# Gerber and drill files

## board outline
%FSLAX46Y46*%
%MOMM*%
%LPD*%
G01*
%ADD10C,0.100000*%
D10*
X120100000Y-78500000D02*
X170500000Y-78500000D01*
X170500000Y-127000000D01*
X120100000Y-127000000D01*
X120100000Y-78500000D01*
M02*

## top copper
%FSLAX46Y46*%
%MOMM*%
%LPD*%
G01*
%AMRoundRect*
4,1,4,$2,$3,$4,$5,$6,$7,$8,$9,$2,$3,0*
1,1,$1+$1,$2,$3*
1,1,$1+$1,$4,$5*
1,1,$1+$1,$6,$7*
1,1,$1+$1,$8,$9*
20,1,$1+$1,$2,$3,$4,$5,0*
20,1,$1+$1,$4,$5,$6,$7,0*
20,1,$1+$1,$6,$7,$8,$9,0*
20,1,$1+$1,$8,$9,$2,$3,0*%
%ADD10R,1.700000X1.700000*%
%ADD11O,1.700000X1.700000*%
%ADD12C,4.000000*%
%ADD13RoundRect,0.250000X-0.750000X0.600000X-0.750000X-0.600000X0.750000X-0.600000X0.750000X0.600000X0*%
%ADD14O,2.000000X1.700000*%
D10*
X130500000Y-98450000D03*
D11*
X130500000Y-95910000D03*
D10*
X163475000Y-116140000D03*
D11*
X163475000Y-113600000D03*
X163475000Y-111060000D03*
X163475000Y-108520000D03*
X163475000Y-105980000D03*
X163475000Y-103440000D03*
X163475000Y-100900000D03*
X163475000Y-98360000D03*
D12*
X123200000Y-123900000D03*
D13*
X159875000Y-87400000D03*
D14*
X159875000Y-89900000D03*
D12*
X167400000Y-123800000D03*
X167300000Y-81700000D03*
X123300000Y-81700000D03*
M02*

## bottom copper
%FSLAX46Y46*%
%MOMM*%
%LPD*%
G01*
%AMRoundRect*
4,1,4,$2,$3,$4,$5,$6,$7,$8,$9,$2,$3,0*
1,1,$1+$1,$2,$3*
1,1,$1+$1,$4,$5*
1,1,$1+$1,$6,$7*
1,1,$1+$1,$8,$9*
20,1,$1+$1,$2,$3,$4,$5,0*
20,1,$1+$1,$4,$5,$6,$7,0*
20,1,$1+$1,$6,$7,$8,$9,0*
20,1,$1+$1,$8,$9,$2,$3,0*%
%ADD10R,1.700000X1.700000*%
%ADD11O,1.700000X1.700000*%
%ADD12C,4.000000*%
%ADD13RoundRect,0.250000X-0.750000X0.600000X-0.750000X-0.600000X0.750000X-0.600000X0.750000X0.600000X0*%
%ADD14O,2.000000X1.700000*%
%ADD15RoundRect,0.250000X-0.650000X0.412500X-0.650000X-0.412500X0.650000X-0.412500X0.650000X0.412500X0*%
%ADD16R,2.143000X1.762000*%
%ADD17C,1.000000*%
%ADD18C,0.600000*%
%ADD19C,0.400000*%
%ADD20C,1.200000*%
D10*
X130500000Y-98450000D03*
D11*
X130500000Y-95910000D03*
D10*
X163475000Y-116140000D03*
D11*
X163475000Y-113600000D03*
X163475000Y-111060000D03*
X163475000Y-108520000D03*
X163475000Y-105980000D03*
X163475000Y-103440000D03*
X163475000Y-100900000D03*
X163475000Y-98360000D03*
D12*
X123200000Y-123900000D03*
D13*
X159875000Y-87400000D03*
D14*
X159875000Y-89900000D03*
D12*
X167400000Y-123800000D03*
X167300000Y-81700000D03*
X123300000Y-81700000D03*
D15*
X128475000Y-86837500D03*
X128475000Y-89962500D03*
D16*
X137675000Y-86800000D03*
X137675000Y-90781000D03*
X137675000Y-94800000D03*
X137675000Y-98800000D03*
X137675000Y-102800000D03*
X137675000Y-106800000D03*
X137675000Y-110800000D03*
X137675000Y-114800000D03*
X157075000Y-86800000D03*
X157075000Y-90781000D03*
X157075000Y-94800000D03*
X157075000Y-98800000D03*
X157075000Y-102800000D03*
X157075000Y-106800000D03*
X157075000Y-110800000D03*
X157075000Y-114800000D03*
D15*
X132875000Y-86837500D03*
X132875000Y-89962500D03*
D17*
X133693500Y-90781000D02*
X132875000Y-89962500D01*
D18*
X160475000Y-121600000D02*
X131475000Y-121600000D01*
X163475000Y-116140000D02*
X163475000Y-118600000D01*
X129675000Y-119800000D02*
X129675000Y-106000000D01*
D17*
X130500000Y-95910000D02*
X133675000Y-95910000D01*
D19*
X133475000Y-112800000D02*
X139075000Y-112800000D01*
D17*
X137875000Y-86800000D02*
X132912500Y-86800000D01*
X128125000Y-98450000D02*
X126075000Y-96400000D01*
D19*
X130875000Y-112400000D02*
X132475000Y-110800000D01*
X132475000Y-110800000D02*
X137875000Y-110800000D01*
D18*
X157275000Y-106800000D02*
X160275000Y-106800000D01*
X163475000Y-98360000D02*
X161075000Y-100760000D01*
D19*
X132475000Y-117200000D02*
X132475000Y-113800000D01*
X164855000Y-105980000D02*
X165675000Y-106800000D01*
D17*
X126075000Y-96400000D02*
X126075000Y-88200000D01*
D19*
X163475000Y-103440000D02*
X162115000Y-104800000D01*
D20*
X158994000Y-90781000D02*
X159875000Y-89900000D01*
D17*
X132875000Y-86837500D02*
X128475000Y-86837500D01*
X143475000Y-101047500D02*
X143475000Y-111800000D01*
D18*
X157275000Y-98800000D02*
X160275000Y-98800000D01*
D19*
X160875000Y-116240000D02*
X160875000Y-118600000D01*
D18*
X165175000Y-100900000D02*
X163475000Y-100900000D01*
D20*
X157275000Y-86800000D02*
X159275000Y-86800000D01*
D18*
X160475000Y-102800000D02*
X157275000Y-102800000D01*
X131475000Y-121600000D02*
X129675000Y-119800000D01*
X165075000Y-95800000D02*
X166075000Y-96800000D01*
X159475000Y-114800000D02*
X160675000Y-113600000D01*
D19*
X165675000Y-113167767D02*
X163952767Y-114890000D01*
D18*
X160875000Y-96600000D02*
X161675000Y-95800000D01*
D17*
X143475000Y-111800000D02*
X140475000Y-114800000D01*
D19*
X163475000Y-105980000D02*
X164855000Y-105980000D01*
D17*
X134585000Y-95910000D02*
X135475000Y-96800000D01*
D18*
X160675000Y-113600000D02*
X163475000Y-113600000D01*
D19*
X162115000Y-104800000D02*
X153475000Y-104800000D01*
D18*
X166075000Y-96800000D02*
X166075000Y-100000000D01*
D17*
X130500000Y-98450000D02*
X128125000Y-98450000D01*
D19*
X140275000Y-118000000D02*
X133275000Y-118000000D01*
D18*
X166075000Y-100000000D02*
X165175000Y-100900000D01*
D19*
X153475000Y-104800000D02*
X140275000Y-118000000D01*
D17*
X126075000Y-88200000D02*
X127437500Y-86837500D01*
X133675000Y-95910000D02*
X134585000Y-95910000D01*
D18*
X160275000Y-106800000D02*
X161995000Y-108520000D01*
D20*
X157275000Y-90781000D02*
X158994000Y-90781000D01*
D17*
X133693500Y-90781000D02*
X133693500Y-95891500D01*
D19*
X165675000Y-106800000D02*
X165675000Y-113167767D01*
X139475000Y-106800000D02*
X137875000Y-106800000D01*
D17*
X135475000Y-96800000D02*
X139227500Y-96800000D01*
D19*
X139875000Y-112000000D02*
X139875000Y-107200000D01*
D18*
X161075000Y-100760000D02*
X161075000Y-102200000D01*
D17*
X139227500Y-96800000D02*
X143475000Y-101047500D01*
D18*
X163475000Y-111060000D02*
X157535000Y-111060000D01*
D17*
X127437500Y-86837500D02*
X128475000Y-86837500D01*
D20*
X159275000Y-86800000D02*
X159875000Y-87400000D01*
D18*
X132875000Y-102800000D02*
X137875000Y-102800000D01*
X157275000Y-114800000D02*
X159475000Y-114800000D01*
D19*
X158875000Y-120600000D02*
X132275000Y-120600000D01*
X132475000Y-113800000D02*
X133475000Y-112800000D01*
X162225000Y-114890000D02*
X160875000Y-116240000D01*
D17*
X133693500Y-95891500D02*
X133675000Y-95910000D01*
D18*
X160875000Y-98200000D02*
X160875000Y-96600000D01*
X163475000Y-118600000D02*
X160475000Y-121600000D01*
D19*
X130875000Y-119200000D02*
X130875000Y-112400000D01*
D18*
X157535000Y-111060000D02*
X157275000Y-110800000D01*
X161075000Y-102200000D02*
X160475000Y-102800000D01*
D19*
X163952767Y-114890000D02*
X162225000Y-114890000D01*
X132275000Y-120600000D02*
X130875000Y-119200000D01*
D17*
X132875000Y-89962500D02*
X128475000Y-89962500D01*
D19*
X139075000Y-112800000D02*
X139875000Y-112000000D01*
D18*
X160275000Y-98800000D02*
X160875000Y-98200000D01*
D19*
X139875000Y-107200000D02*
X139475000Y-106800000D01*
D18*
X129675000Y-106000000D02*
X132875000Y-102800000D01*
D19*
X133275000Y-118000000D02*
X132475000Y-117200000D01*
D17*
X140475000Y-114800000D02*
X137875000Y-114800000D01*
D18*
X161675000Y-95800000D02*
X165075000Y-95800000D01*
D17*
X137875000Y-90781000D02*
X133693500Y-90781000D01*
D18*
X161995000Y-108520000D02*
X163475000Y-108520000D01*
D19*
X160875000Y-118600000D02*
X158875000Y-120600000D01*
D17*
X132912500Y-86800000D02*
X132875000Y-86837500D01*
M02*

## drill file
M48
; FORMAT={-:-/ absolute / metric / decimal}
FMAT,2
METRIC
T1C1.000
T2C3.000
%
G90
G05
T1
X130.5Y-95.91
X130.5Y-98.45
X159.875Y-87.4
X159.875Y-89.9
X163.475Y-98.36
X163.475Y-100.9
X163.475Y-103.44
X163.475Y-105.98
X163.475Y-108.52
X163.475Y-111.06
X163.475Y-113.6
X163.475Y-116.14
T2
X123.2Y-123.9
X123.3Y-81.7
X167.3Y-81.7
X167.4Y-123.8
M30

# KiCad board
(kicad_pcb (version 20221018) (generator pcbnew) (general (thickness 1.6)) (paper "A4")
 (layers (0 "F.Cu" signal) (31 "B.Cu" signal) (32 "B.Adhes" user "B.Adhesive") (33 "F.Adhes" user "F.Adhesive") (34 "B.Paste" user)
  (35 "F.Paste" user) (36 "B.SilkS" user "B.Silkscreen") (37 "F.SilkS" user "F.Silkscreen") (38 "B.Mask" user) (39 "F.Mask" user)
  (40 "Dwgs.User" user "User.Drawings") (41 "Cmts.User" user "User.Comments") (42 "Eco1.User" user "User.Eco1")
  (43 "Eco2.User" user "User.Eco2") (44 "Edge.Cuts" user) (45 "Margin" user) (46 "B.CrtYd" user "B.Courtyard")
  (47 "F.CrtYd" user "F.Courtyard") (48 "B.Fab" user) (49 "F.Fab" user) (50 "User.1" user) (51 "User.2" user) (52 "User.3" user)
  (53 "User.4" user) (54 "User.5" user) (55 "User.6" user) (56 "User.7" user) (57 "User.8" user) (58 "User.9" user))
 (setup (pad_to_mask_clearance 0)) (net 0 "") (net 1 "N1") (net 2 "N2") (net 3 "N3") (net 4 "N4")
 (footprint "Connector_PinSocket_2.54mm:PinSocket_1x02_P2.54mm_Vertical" (layer "F.Cu") (at 130.5 98.45 180)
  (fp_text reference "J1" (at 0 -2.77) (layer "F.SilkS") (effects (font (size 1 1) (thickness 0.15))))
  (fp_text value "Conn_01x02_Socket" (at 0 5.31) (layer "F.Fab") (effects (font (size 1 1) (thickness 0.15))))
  (pad "1" thru_hole rect (at 0 0 180) (size 1.7 1.7) (drill 1) (layers "*.Cu" "*.Mask"))
  (pad "2" thru_hole oval (at 0 2.54 180) (size 1.7 1.7) (drill 1) (layers "*.Cu" "*.Mask")))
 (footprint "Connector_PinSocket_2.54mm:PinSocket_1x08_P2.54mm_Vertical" (layer "F.Cu") (at 163.475 116.14 180)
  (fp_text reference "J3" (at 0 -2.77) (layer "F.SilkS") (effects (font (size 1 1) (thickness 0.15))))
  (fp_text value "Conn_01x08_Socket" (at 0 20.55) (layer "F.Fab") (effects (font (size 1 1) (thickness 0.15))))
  (pad "1" thru_hole rect (at 0 0 180) (size 1.7 1.7) (drill 1) (layers "*.Cu" "*.Mask"))
  (pad "2" thru_hole oval (at 0 2.54 180) (size 1.7 1.7) (drill 1) (layers "*.Cu" "*.Mask"))
  (pad "3" thru_hole oval (at 0 5.08 180) (size 1.7 1.7) (drill 1) (layers "*.Cu" "*.Mask"))
  (pad "4" thru_hole oval (at 0 7.62 180) (size 1.7 1.7) (drill 1) (layers "*.Cu" "*.Mask"))
  (pad "5" thru_hole oval (at 0 10.16 180) (size 1.7 1.7) (drill 1) (layers "*.Cu" "*.Mask"))
  (pad "6" thru_hole oval (at 0 12.7 180) (size 1.7 1.7) (drill 1) (layers "*.Cu" "*.Mask"))
  (pad "7" thru_hole oval (at 0 15.24 180) (size 1.7 1.7) (drill 1) (layers "*.Cu" "*.Mask"))
  (pad "8" thru_hole oval (at 0 17.78 180) (size 1.7 1.7) (drill 1) (layers "*.Cu" "*.Mask")))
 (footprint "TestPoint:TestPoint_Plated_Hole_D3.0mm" (layer "F.Cu") (at 123.2 123.9)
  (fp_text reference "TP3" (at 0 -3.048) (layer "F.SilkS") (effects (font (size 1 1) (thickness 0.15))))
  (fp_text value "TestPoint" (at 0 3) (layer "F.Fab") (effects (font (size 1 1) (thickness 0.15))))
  (pad "1" thru_hole circle (at 0 0) (size 4 4) (drill 3) (layers "*.Cu" "*.Mask") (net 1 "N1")))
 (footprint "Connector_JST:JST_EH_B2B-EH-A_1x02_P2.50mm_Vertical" (layer "F.Cu") (at 159.875 87.4 -90)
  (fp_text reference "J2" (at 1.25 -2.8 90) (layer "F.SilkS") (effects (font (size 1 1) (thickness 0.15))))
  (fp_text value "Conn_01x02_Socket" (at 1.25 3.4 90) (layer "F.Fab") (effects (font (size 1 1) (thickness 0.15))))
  (pad "1" thru_hole roundrect (at 0 0 270) (size 1.7 2) (drill 1) (layers "*.Cu" "*.Mask") (roundrect_rratio 0.1470588235))
  (pad "2" thru_hole oval (at 2.5 0 270) (size 1.7 2) (drill 1) (layers "*.Cu" "*.Mask")))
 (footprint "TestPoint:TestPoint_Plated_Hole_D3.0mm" (layer "F.Cu") (at 167.4 123.8)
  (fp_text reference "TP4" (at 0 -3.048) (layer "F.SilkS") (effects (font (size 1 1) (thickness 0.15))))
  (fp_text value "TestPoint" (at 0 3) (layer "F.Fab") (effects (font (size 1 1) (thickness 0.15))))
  (pad "1" thru_hole circle (at 0 0) (size 4 4) (drill 3) (layers "*.Cu" "*.Mask") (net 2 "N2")))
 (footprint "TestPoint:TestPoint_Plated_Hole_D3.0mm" (layer "F.Cu") (at 167.3 81.7)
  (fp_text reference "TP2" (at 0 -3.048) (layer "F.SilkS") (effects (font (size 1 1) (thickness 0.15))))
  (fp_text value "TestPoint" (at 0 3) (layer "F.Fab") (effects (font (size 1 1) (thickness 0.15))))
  (pad "1" thru_hole circle (at 0 0) (size 4 4) (drill 3) (layers "*.Cu" "*.Mask") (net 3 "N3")))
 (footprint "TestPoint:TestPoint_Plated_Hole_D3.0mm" (layer "F.Cu") (at 123.3 81.7)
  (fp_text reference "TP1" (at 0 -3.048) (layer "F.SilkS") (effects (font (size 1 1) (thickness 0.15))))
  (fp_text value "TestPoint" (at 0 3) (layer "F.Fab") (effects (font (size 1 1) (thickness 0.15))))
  (pad "1" thru_hole circle (at 0 0) (size 4 4) (drill 3) (layers "*.Cu" "*.Mask") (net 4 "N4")))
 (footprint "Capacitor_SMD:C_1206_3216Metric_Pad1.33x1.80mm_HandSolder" (layer "B.Cu") (at 128.475 88.4 -90)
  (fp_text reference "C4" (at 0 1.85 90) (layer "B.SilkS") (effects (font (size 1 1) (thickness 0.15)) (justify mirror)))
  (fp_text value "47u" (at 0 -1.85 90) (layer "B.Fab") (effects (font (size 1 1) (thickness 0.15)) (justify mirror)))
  (pad "1" smd roundrect (at -1.5625 0 270) (size 1.325 1.8) (layers "B.Cu" "B.Paste" "B.Mask") (roundrect_rratio 0.1886792453))
  (pad "2" smd roundrect (at 1.5625 0 270) (size 1.325 1.8) (layers "B.Cu" "B.Paste" "B.Mask") (roundrect_rratio 0.1886792453)))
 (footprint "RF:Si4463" (layer "B.Cu") (at 147.375 100.8 -90)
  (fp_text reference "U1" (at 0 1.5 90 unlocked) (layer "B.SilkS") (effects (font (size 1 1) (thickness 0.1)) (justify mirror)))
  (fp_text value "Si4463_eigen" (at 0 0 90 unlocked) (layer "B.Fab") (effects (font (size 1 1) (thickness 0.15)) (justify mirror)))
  (pad "1" smd rect (at -14 9.7 180) (size 2.143 1.762) (layers "B.Cu" "B.Paste" "B.Mask") (thermal_bridge_angle 45))
  (pad "2" smd rect (at -10.019 9.7 180) (size 2.143 1.762) (layers "B.Cu" "B.Paste" "B.Mask") (thermal_bridge_angle 45))
  (pad "3" smd rect (at -6 9.7 180) (size 2.143 1.762) (layers "B.Cu" "B.Paste" "B.Mask") (thermal_bridge_angle 45))
  (pad "4" smd rect (at -2 9.7 180) (size 2.143 1.762) (layers "B.Cu" "B.Paste" "B.Mask") (thermal_bridge_angle 45))
  (pad "5" smd rect (at 2 9.7 180) (size 2.143 1.762) (layers "B.Cu" "B.Paste" "B.Mask") (thermal_bridge_angle 45))
  (pad "6" smd rect (at 6 9.7 180) (size 2.143 1.762) (layers "B.Cu" "B.Paste" "B.Mask") (thermal_bridge_angle 45))
  (pad "7" smd rect (at 10 9.7 180) (size 2.143 1.762) (layers "B.Cu" "B.Paste" "B.Mask") (thermal_bridge_angle 45))
  (pad "8" smd rect (at 14 9.7 180) (size 2.143 1.762) (layers "B.Cu" "B.Paste" "B.Mask") (thermal_bridge_angle 45))
  (pad "9" smd rect (at -14 -9.7 180) (size 2.143 1.762) (layers "B.Cu" "B.Paste" "B.Mask") (thermal_bridge_angle 45))
  (pad "10" smd rect (at -10.019 -9.7 180) (size 2.143 1.762) (layers "B.Cu" "B.Paste" "B.Mask") (thermal_bridge_angle 45))
  (pad "11" smd rect (at -6 -9.7 180) (size 2.143 1.762) (layers "B.Cu" "B.Paste" "B.Mask") (thermal_bridge_angle 45))
  (pad "12" smd rect (at -2 -9.7 180) (size 2.143 1.762) (layers "B.Cu" "B.Paste" "B.Mask") (thermal_bridge_angle 45))
  (pad "13" smd rect (at 2 -9.7 180) (size 2.143 1.762) (layers "B.Cu" "B.Paste" "B.Mask") (thermal_bridge_angle 45))
  (pad "14" smd rect (at 6 -9.7 180) (size 2.143 1.762) (layers "B.Cu" "B.Paste" "B.Mask") (thermal_bridge_angle 45))
  (pad "15" smd rect (at 10 -9.7 180) (size 2.143 1.762) (layers "B.Cu" "B.Paste" "B.Mask") (thermal_bridge_angle 45))
  (pad "16" smd rect (at 14 -9.7 180) (size 2.143 1.762) (layers "B.Cu" "B.Paste" "B.Mask") (thermal_bridge_angle 45)))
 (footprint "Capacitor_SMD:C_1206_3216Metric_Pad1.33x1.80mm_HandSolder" (layer "B.Cu") (at 132.875 88.4 -90)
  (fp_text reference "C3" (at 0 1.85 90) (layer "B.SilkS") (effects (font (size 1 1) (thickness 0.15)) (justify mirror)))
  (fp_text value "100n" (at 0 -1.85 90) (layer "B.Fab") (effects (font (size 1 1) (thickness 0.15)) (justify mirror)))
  (pad "1" smd roundrect (at -1.5625 0 270) (size 1.325 1.8) (layers "B.Cu" "B.Paste" "B.Mask") (roundrect_rratio 0.1886792453))
  (pad "2" smd roundrect (at 1.5625 0 270) (size 1.325 1.8) (layers "B.Cu" "B.Paste" "B.Mask") (roundrect_rratio 0.1886792453)))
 (gr_rect (start 120.1 78.5) (end 170.5 127) (stroke (width 0.1) (type default)) (fill none) (layer "Edge.Cuts"))
 (segment (start 133.6935 90.781) (end 132.875 89.9625) (width 1) (layer "B.Cu") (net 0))
 (segment (start 160.475 121.6) (end 131.475 121.6) (width 0.6) (layer "B.Cu") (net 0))
 (segment (start 163.475 116.14) (end 163.475 118.6) (width 0.6) (layer "B.Cu") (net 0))
 (segment (start 129.675 119.8) (end 129.675 106) (width 0.6) (layer "B.Cu") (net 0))
 (segment (start 130.5 95.91) (end 133.675 95.91) (width 1) (layer "B.Cu") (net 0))
 (segment (start 133.475 112.8) (end 139.075 112.8) (width 0.4) (layer "B.Cu") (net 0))
 (segment (start 137.875 86.8) (end 132.9125 86.8) (width 1) (layer "B.Cu") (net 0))
 (segment (start 128.125 98.45) (end 126.075 96.4) (width 1) (layer "B.Cu") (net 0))
 (segment (start 130.875 112.4) (end 132.475 110.8) (width 0.4) (layer "B.Cu") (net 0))
 (segment (start 132.475 110.8) (end 137.875 110.8) (width 0.4) (layer "B.Cu") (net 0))
 (segment (start 157.275 106.8) (end 160.275 106.8) (width 0.6) (layer "B.Cu") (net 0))
 (segment (start 163.475 98.36) (end 161.075 100.76) (width 0.6) (layer "B.Cu") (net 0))
 (segment (start 132.475 117.2) (end 132.475 113.8) (width 0.4) (layer "B.Cu") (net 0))
 (segment (start 164.855 105.98) (end 165.675 106.8) (width 0.4) (layer "B.Cu") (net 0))
 (segment (start 126.075 96.4) (end 126.075 88.2) (width 1) (layer "B.Cu") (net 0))
 (segment (start 163.475 103.44) (end 162.115 104.8) (width 0.4) (layer "B.Cu") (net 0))
 (segment (start 158.994 90.781) (end 159.875 89.9) (width 1.2) (layer "B.Cu") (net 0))
 (segment (start 132.875 86.8375) (end 128.475 86.8375) (width 1) (layer "B.Cu") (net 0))
 (segment (start 143.475 101.0475) (end 143.475 111.8) (width 1) (layer "B.Cu") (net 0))
 (segment (start 157.275 98.8) (end 160.275 98.8) (width 0.6) (layer "B.Cu") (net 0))
 (segment (start 160.875 116.24) (end 160.875 118.6) (width 0.4) (layer "B.Cu") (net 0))
 (segment (start 165.175 100.9) (end 163.475 100.9) (width 0.6) (layer "B.Cu") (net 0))
 (segment (start 157.275 86.8) (end 159.275 86.8) (width 1.2) (layer "B.Cu") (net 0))
 (segment (start 160.475 102.8) (end 157.275 102.8) (width 0.6) (layer "B.Cu") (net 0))
 (segment (start 131.475 121.6) (end 129.675 119.8) (width 0.6) (layer "B.Cu") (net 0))
 (segment (start 165.075 95.8) (end 166.075 96.8) (width 0.6) (layer "B.Cu") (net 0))
 (segment (start 159.475 114.8) (end 160.675 113.6) (width 0.6) (layer "B.Cu") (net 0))
 (segment (start 165.675 113.167767) (end 163.952767 114.89) (width 0.4) (layer "B.Cu") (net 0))
 (segment (start 160.875 96.6) (end 161.675 95.8) (width 0.6) (layer "B.Cu") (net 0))
 (segment (start 143.475 111.8) (end 140.475 114.8) (width 1) (layer "B.Cu") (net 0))
 (segment (start 163.475 105.98) (end 164.855 105.98) (width 0.4) (layer "B.Cu") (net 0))
 (segment (start 134.585 95.91) (end 135.475 96.8) (width 1) (layer "B.Cu") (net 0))
 (segment (start 160.675 113.6) (end 163.475 113.6) (width 0.6) (layer "B.Cu") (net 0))
 (segment (start 162.115 104.8) (end 153.475 104.8) (width 0.4) (layer "B.Cu") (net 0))
 (segment (start 166.075 96.8) (end 166.075 100) (width 0.6) (layer "B.Cu") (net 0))
 (segment (start 130.5 98.45) (end 128.125 98.45) (width 1) (layer "B.Cu") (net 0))
 (segment (start 140.275 118) (end 133.275 118) (width 0.4) (layer "B.Cu") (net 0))
 (segment (start 166.075 100) (end 165.175 100.9) (width 0.6) (layer "B.Cu") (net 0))
 (segment (start 153.475 104.8) (end 140.275 118) (width 0.4) (layer "B.Cu") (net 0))
 (segment (start 126.075 88.2) (end 127.4375 86.8375) (width 1) (layer "B.Cu") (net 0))
 (segment (start 133.675 95.91) (end 134.585 95.91) (width 1) (layer "B.Cu") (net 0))
 (segment (start 160.275 106.8) (end 161.995 108.52) (width 0.6) (layer "B.Cu") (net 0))
 (segment (start 157.275 90.781) (end 158.994 90.781) (width 1.2) (layer "B.Cu") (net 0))
 (segment (start 133.6935 90.781) (end 133.6935 95.8915) (width 1) (layer "B.Cu") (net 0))
 (segment (start 165.675 106.8) (end 165.675 113.167767) (width 0.4) (layer "B.Cu") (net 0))
 (segment (start 139.475 106.8) (end 137.875 106.8) (width 0.4) (layer "B.Cu") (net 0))
 (segment (start 135.475 96.8) (end 139.2275 96.8) (width 1) (layer "B.Cu") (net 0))
 (segment (start 139.875 112) (end 139.875 107.2) (width 0.4) (layer "B.Cu") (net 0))
 (segment (start 161.075 100.76) (end 161.075 102.2) (width 0.6) (layer "B.Cu") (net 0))
 (segment (start 139.2275 96.8) (end 143.475 101.0475) (width 1) (layer "B.Cu") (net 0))
 (segment (start 163.475 111.06) (end 157.535 111.06) (width 0.6) (layer "B.Cu") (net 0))
 (segment (start 127.4375 86.8375) (end 128.475 86.8375) (width 1) (layer "B.Cu") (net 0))
 (segment (start 159.275 86.8) (end 159.875 87.4) (width 1.2) (layer "B.Cu") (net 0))
 (segment (start 132.875 102.8) (end 137.875 102.8) (width 0.6) (layer "B.Cu") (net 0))
 (segment (start 157.275 114.8) (end 159.475 114.8) (width 0.6) (layer "B.Cu") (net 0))
 (segment (start 158.875 120.6) (end 132.275 120.6) (width 0.4) (layer "B.Cu") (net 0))
 (segment (start 132.475 113.8) (end 133.475 112.8) (width 0.4) (layer "B.Cu") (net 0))
 (segment (start 162.225 114.89) (end 160.875 116.24) (width 0.4) (layer "B.Cu") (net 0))
 (segment (start 133.6935 95.8915) (end 133.675 95.91) (width 1) (layer "B.Cu") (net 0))
 (segment (start 160.875 98.2) (end 160.875 96.6) (width 0.6) (layer "B.Cu") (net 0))
 (segment (start 163.475 118.6) (end 160.475 121.6) (width 0.6) (layer "B.Cu") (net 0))
 (segment (start 130.875 119.2) (end 130.875 112.4) (width 0.4) (layer "B.Cu") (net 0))
 (segment (start 157.535 111.06) (end 157.275 110.8) (width 0.6) (layer "B.Cu") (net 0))
 (segment (start 161.075 102.2) (end 160.475 102.8) (width 0.6) (layer "B.Cu") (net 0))
 (segment (start 163.952767 114.89) (end 162.225 114.89) (width 0.4) (layer "B.Cu") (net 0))
 (segment (start 132.275 120.6) (end 130.875 119.2) (width 0.4) (layer "B.Cu") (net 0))
 (segment (start 132.875 89.9625) (end 128.475 89.9625) (width 1) (layer "B.Cu") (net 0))
 (segment (start 139.075 112.8) (end 139.875 112) (width 0.4) (layer "B.Cu") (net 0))
 (segment (start 160.275 98.8) (end 160.875 98.2) (width 0.6) (layer "B.Cu") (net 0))
 (segment (start 139.875 107.2) (end 139.475 106.8) (width 0.4) (layer "B.Cu") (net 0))
 (segment (start 129.675 106) (end 132.875 102.8) (width 0.6) (layer "B.Cu") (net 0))
 (segment (start 133.275 118) (end 132.475 117.2) (width 0.4) (layer "B.Cu") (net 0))
 (segment (start 140.475 114.8) (end 137.875 114.8) (width 1) (layer "B.Cu") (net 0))
 (segment (start 161.675 95.8) (end 165.075 95.8) (width 0.6) (layer "B.Cu") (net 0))
 (segment (start 137.875 90.781) (end 133.6935 90.781) (width 1) (layer "B.Cu") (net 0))
 (segment (start 161.995 108.52) (end 163.475 108.52) (width 0.6) (layer "B.Cu") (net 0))
 (segment (start 160.875 118.6) (end 158.875 120.6) (width 0.4) (layer "B.Cu") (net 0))
 (segment (start 132.9125 86.8) (end 132.875 86.8375) (width 1) (layer "B.Cu") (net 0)))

